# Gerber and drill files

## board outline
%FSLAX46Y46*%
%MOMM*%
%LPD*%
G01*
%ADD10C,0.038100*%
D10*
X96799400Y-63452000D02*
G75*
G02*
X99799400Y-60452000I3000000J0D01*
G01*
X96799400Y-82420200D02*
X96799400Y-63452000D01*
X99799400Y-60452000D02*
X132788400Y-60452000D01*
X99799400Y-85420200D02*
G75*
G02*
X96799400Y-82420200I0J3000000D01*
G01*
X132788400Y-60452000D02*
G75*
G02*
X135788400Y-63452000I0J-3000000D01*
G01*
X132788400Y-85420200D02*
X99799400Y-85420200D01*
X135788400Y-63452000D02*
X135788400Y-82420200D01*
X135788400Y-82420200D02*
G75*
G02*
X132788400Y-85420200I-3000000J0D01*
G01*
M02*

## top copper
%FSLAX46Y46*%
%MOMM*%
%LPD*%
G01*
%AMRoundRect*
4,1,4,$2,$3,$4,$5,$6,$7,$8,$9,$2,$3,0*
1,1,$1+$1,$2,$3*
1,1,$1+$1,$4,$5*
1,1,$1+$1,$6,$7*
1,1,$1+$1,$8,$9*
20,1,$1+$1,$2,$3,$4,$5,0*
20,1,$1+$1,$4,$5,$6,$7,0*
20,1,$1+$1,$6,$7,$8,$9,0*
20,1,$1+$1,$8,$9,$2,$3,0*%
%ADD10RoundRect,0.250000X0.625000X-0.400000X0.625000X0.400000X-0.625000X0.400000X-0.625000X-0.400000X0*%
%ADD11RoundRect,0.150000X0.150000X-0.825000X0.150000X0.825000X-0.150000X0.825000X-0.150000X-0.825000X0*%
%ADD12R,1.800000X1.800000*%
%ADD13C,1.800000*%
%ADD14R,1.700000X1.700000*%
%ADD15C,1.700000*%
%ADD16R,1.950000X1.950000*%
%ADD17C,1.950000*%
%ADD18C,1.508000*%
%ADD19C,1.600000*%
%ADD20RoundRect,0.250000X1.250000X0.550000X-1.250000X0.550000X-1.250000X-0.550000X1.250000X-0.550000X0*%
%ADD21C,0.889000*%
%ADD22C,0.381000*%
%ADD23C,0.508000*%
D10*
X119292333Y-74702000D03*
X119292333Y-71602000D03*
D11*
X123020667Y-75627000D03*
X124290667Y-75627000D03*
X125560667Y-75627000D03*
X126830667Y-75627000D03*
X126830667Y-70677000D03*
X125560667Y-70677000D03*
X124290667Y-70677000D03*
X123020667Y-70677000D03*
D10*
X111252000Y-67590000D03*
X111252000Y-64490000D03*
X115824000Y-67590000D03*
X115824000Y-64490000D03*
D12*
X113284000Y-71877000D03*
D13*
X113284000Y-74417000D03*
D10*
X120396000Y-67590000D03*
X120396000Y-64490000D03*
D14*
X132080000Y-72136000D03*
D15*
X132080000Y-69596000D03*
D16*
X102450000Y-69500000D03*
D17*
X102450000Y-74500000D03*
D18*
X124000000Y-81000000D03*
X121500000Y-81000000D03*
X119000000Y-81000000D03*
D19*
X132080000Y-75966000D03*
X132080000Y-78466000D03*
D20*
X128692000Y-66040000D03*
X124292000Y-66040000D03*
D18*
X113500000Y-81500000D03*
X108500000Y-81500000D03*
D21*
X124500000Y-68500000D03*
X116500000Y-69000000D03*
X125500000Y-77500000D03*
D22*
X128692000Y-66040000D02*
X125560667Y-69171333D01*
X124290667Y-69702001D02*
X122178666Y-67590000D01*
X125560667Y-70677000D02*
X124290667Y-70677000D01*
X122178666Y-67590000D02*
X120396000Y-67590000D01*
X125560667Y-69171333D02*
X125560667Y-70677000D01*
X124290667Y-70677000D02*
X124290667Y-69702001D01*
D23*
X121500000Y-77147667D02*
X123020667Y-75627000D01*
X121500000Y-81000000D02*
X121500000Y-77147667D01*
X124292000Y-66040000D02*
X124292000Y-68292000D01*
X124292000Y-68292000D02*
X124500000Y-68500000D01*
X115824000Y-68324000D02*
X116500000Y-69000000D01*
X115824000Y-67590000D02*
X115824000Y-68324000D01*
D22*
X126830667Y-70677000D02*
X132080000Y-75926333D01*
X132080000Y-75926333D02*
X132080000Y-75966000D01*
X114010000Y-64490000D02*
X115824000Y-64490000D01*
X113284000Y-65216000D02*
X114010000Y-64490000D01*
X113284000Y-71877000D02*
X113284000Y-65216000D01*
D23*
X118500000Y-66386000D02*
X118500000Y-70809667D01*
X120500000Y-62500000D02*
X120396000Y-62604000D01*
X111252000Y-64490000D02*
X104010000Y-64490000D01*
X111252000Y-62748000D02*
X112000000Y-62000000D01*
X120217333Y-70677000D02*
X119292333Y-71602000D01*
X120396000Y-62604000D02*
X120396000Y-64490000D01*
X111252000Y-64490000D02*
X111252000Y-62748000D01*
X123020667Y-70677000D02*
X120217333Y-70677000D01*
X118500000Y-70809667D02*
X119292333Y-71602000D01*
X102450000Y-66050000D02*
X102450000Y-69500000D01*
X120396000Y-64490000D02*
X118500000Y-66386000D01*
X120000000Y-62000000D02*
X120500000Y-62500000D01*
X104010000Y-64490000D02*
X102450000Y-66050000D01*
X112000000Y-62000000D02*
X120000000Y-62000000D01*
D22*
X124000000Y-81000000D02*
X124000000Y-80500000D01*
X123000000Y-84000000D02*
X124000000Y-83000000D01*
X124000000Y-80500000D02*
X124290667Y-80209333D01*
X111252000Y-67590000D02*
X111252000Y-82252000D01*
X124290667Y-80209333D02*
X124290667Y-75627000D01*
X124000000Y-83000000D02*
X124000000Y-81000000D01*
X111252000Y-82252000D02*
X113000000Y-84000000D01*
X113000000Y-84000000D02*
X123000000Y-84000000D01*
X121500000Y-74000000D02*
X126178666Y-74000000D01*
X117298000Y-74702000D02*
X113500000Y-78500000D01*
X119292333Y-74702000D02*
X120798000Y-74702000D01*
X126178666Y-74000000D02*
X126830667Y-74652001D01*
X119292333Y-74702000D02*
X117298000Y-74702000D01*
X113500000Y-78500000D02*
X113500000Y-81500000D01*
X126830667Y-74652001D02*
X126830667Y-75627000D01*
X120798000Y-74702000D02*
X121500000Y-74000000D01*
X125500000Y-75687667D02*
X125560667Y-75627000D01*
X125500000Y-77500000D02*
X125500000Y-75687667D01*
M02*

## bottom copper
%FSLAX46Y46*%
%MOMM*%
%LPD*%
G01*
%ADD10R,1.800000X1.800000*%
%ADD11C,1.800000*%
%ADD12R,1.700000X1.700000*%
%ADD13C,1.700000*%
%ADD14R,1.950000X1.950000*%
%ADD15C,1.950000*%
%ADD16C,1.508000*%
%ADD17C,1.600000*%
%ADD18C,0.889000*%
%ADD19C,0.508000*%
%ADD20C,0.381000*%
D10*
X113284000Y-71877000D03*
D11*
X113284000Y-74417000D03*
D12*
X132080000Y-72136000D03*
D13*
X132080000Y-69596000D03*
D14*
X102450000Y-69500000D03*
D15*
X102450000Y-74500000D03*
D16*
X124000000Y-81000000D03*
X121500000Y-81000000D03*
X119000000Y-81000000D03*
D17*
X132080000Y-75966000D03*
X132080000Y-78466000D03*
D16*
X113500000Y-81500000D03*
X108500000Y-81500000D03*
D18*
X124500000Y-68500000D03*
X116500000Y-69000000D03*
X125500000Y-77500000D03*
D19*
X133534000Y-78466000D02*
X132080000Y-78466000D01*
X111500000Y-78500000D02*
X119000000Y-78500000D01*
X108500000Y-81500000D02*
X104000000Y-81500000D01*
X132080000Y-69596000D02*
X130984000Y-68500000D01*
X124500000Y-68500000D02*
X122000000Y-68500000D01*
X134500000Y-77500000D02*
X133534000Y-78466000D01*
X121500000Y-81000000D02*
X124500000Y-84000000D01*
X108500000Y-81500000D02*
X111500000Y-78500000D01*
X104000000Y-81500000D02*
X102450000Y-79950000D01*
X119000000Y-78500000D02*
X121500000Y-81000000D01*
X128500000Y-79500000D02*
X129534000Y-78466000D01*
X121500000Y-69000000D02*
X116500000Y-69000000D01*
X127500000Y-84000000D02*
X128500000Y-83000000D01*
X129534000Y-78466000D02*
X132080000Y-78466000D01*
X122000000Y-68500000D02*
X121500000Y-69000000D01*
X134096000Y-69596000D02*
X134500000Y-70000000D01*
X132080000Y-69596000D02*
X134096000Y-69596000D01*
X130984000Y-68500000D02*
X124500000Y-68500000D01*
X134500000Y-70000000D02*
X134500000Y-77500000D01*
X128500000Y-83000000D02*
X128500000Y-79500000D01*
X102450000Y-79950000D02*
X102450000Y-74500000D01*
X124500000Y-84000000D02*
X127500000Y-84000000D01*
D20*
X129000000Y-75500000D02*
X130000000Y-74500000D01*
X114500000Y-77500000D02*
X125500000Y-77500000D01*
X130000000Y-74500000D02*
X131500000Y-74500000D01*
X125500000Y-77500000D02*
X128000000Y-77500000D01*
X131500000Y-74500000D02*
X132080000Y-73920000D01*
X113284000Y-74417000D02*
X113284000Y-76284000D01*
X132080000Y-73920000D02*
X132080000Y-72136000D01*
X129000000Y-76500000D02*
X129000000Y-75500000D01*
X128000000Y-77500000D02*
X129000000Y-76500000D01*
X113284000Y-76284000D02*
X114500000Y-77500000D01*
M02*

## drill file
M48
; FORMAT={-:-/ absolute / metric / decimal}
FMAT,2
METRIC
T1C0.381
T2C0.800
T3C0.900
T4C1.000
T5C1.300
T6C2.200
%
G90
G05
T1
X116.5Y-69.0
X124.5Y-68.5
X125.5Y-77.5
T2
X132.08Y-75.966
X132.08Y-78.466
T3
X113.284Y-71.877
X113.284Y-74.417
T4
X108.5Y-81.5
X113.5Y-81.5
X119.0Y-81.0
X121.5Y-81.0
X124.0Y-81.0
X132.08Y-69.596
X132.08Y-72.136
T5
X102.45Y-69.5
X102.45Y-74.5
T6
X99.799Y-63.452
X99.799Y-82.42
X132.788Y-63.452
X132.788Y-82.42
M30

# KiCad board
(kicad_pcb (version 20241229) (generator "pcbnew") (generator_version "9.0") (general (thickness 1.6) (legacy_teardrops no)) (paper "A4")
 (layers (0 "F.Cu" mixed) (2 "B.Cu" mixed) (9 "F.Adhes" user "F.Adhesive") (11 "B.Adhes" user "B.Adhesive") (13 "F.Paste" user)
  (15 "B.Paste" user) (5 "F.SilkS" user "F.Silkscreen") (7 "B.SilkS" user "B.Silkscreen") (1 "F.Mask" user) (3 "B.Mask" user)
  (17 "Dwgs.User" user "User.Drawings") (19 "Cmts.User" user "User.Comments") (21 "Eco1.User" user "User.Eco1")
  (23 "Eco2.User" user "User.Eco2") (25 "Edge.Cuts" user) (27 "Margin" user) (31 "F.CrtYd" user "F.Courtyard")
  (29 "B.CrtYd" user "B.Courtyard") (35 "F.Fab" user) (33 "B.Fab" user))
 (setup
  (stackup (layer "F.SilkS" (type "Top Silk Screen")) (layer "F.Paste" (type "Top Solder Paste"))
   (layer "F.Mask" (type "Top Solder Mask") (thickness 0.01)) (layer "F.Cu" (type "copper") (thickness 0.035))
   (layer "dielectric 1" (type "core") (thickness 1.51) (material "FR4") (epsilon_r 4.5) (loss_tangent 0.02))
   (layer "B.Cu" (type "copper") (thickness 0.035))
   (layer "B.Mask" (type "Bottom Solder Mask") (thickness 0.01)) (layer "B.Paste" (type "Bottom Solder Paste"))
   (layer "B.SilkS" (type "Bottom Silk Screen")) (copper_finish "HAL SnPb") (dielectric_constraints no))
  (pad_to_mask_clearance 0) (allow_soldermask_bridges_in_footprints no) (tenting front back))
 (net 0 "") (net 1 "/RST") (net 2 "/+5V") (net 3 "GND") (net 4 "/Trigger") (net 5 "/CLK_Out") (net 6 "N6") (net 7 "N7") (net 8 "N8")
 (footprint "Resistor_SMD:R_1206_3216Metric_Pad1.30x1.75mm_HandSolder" (layer "F.Cu") (at 119.292333 73.152 90)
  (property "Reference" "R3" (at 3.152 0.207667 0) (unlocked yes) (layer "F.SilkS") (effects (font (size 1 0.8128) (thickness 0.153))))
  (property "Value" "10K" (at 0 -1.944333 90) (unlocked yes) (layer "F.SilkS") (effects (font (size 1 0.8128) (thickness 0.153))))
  (pad "1" smd roundrect (at -1.55 0 90) (size 1.3 1.75) (layers "F.Cu" "F.Mask" "F.Paste") (roundrect_rratio 0.192308) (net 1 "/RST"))
  (pad "2" smd roundrect (at 1.55 0 90) (size 1.3 1.75) (layers "F.Cu" "F.Mask" "F.Paste") (roundrect_rratio 0.192308) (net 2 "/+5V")))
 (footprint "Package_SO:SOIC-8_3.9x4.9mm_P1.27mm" (layer "F.Cu") (at 124.925667 73.152 90)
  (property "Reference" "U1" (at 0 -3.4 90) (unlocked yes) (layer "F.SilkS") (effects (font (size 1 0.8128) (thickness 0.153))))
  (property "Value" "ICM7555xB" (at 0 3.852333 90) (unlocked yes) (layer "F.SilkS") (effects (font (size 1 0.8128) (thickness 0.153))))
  (pad "1" smd roundrect (at -2.475 -1.905 90) (size 1.95 0.6) (layers "F.Cu" "F.Mask" "F.Paste") (roundrect_rratio 0.25) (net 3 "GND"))
  (pad "2" smd roundrect (at -2.475 -0.635 90) (size 1.95 0.6) (layers "F.Cu" "F.Mask" "F.Paste") (roundrect_rratio 0.25) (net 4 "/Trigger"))
  (pad "3" smd roundrect (at -2.475 0.635 90) (size 1.95 0.6) (layers "F.Cu" "F.Mask" "F.Paste") (roundrect_rratio 0.25) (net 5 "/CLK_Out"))
  (pad "4" smd roundrect (at -2.475 1.905 90) (size 1.95 0.6) (layers "F.Cu" "F.Mask" "F.Paste") (roundrect_rratio 0.25) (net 1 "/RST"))
  (pad "5" smd roundrect (at 2.475 1.905 90) (size 1.95 0.6) (layers "F.Cu" "F.Mask" "F.Paste") (roundrect_rratio 0.25) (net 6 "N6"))
  (pad "6" smd roundrect (at 2.475 0.635 90) (size 1.95 0.6) (layers "F.Cu" "F.Mask" "F.Paste") (roundrect_rratio 0.25) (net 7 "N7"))
  (pad "7" smd roundrect (at 2.475 -0.635 90) (size 1.95 0.6) (layers "F.Cu" "F.Mask" "F.Paste") (roundrect_rratio 0.25) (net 7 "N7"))
  (pad "8" smd roundrect (at 2.475 -1.905 90) (size 1.95 0.6) (layers "F.Cu" "F.Mask" "F.Paste") (roundrect_rratio 0.25) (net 2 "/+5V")))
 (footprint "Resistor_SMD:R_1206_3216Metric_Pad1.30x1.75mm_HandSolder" (layer "F.Cu") (at 111.252 66.04 90)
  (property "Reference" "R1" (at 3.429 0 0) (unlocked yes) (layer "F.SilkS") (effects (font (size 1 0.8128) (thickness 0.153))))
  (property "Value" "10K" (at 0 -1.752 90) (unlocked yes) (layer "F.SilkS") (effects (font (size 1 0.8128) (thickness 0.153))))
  (pad "1" smd roundrect (at -1.55 0 90) (size 1.3 1.75) (layers "F.Cu" "F.Mask" "F.Paste") (roundrect_rratio 0.192308) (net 4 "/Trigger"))
  (pad "2" smd roundrect (at 1.55 0 90) (size 1.3 1.75) (layers "F.Cu" "F.Mask" "F.Paste") (roundrect_rratio 0.192308) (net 2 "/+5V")))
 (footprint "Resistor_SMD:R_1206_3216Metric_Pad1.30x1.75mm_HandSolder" (layer "F.Cu") (at 115.824 66.04 90)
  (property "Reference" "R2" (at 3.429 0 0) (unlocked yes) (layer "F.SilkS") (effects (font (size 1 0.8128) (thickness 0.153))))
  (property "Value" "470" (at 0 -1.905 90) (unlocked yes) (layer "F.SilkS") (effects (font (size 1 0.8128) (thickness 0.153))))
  (pad "1" smd roundrect (at -1.55 0 90) (size 1.3 1.75) (layers "F.Cu" "F.Mask" "F.Paste") (roundrect_rratio 0.192308) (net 3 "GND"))
  (pad "2" smd roundrect (at 1.55 0 90) (size 1.3 1.75) (layers "F.Cu" "F.Mask" "F.Paste") (roundrect_rratio 0.192308) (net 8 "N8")))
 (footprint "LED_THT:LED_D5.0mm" (layer "F.Cu") (at 113.284 71.877 -90)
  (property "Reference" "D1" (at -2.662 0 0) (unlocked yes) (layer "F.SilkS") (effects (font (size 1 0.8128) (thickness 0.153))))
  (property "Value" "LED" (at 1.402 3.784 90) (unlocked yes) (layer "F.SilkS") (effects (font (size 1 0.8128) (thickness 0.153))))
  (pad "1" thru_hole rect (at 0 0 270) (size 1.8 1.8) (drill 0.9) (layers "*.Cu" "*.Mask") (remove_unused_layers no) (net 8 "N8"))
  (pad "2" thru_hole circle (at 2.54 0 270) (size 1.8 1.8) (drill 0.9) (layers "*.Cu" "*.Mask") (remove_unused_layers no) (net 5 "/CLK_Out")))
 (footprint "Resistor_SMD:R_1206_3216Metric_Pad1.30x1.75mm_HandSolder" (layer "F.Cu") (at 120.396 66.04 90)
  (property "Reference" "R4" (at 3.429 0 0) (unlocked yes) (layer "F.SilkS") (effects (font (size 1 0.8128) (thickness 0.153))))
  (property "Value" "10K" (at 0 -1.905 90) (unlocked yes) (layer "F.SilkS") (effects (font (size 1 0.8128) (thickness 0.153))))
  (pad "1" smd roundrect (at -1.55 0 90) (size 1.3 1.75) (layers "F.Cu" "F.Mask" "F.Paste") (roundrect_rratio 0.192308) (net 7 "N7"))
  (pad "2" smd roundrect (at 1.55 0 90) (size 1.3 1.75) (layers "F.Cu" "F.Mask" "F.Paste") (roundrect_rratio 0.192308) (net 2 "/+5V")))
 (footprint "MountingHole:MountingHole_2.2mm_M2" (layer "F.Cu") (at 99.7994 63.452)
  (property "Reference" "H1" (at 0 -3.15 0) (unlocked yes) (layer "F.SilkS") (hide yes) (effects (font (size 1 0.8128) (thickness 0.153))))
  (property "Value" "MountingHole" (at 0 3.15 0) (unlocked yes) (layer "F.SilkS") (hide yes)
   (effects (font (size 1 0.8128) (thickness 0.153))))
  (pad "" np_thru_hole circle (at 0 0) (size 2.2 2.2) (drill 2.2) (layers "*.Cu" "*.Mask")))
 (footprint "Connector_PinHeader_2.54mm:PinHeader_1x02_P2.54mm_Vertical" (layer "F.Cu") (at 132.08 72.136 180)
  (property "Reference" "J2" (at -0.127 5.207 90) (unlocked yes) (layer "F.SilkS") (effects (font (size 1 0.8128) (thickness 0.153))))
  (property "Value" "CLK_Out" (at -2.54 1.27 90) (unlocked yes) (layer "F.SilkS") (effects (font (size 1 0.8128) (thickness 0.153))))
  (pad "1" thru_hole rect (at 0 0 180) (size 1.7 1.7) (drill 1) (layers "*.Cu" "*.Mask") (remove_unused_layers no) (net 5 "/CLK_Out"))
  (pad "2" thru_hole circle (at 0 2.54 180) (size 1.7 1.7) (drill 1) (layers "*.Cu" "*.Mask") (remove_unused_layers no) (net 3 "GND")))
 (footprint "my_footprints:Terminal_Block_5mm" (layer "F.Cu") (at 102.45 72 -90)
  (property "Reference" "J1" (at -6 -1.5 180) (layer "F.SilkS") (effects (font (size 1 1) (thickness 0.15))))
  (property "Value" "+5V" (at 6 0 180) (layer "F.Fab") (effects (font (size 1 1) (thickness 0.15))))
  (pad "1" thru_hole rect (at -2.5 0 270) (size 1.95 1.95) (drill 1.3) (layers "*.Cu" "*.Mask") (remove_unused_layers no) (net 2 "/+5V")
   (solder_mask_margin 0.102))
  (pad "2" thru_hole circle (at 2.5 0 270) (size 1.95 1.95) (drill 1.3) (layers "*.Cu" "*.Mask") (remove_unused_layers no) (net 3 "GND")
   (solder_mask_margin 0.102)))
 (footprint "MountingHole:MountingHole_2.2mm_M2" (layer "F.Cu") (at 132.7884 82.4202)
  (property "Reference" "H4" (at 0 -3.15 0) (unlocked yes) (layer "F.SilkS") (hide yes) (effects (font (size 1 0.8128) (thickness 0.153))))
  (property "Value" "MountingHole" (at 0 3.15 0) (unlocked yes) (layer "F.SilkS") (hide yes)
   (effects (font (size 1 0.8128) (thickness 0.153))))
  (pad "" np_thru_hole circle (at 0 0) (size 2.2 2.2) (drill 2.2) (layers "*.Cu" "*.Mask")))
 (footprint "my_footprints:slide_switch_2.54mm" (layer "F.Cu") (at 121.5 81 180)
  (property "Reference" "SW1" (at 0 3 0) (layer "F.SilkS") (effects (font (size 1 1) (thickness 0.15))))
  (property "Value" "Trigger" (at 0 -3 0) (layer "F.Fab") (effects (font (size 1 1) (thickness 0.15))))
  (pad "1" thru_hole circle (at -2.5 0 180) (size 1.508 1.508) (drill 1) (layers "*.Cu" "*.Mask") (remove_unused_layers no)
   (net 4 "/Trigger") (solder_mask_margin 0.102))
  (pad "2" thru_hole circle (at 0 0 180) (size 1.508 1.508) (drill 1) (layers "*.Cu" "*.Mask") (remove_unused_layers no) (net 3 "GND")
   (solder_mask_margin 0.102))
  (pad "3" thru_hole circle (at 2.5 0 180) (size 1.508 1.508) (drill 1) (layers "*.Cu" "*.Mask") (remove_unused_layers no)
   (solder_mask_margin 0.102)))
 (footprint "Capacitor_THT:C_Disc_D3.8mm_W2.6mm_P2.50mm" (layer "F.Cu") (at 132.08 75.966 -90)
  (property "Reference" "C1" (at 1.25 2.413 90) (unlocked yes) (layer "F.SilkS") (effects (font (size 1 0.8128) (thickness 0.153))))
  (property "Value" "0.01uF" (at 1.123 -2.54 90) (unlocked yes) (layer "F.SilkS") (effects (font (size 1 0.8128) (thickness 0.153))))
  (pad "1" thru_hole circle (at 0 0 270) (size 1.6 1.6) (drill 0.8) (layers "*.Cu" "*.Mask") (remove_unused_layers no) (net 6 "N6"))
  (pad "2" thru_hole circle (at 2.5 0 270) (size 1.6 1.6) (drill 0.8) (layers "*.Cu" "*.Mask") (remove_unused_layers no) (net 3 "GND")))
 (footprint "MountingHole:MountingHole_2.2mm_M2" (layer "F.Cu") (at 132.7884 63.452)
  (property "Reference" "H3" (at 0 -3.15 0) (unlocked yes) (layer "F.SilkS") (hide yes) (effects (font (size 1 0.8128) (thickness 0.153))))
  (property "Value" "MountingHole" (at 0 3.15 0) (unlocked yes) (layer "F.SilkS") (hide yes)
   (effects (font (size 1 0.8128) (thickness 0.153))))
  (pad "" np_thru_hole circle (at 0 0) (size 2.2 2.2) (drill 2.2) (layers "*.Cu" "*.Mask")))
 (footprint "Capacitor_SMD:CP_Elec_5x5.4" (layer "F.Cu") (at 126.492 66.04 180)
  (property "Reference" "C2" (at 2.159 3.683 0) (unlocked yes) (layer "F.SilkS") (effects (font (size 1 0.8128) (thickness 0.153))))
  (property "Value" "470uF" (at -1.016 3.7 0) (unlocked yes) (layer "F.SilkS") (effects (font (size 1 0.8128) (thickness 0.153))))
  (pad "1" smd roundrect (at -2.2 0 180) (size 3 1.6) (layers "F.Cu" "F.Mask" "F.Paste") (roundrect_rratio 0.15625) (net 7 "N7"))
  (pad "2" smd roundrect (at 2.2 0 180) (size 3 1.6) (layers "F.Cu" "F.Mask" "F.Paste") (roundrect_rratio 0.15625) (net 3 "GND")))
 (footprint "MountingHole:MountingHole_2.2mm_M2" (layer "F.Cu") (at 99.7994 82.4202)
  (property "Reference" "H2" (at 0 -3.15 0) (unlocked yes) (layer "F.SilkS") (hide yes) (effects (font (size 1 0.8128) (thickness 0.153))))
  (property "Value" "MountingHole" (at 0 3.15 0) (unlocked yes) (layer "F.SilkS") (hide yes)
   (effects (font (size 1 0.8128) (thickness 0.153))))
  (pad "" np_thru_hole circle (at 0 0) (size 2.2 2.2) (drill 2.2) (layers "*.Cu" "*.Mask")))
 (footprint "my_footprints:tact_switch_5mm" (layer "F.Cu") (at 111 81.5 180)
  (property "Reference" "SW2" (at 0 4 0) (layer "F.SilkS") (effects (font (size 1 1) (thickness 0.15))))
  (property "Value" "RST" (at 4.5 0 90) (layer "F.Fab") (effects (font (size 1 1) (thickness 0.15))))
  (pad "1" thru_hole circle (at -2.5 0 180) (size 1.508 1.508) (drill 1) (layers "*.Cu" "*.Mask") (remove_unused_layers no) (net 1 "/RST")
   (solder_mask_margin 0.102))
  (pad "2" thru_hole circle (at 2.5 0 180) (size 1.508 1.508) (drill 1) (layers "*.Cu" "*.Mask") (remove_unused_layers no) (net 3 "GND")
   (solder_mask_margin 0.102)))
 (gr_arc (start 96.7994 63.452) (mid 97.67808 61.33068) (end 99.7994 60.452) (stroke (width 0.0381) (type default)) (layer "Edge.Cuts"))
 (gr_line (start 96.7994 82.4202) (end 96.7994 63.452) (stroke (width 0.0381) (type default)) (layer "Edge.Cuts"))
 (gr_line (start 99.7994 60.452) (end 132.7884 60.452) (stroke (width 0.0381) (type default)) (layer "Edge.Cuts"))
 (gr_arc (start 99.7994 85.4202) (mid 97.67808 84.54152) (end 96.7994 82.4202) (stroke (width 0.0381) (type default)) (layer "Edge.Cuts"))
 (gr_arc (start 132.7884 60.452) (mid 134.90972 61.33068) (end 135.7884 63.452) (stroke (width 0.0381) (type default)) (layer "Edge.Cuts"))
 (gr_line (start 132.7884 85.4202) (end 99.7994 85.4202) (stroke (width 0.0381) (type default)) (layer "Edge.Cuts"))
 (gr_line (start 135.7884 63.452) (end 135.7884 82.4202) (stroke (width 0.0381) (type default)) (layer "Edge.Cuts"))
 (gr_arc (start 135.7884 82.4202) (mid 134.90972 84.54152) (end 132.7884 85.4202) (stroke (width 0.0381) (type default)) (layer "Edge.Cuts"))
 (segment (start 128.692 66.04) (end 125.560667 69.171333) (width 0.381) (layer "F.Cu") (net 7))
 (segment (start 124.290667 69.702001) (end 122.178666 67.59) (width 0.381) (layer "F.Cu") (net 7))
 (segment (start 125.560667 70.677) (end 124.290667 70.677) (width 0.381) (layer "F.Cu") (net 7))
 (segment (start 122.178666 67.59) (end 120.396 67.59) (width 0.381) (layer "F.Cu") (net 7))
 (segment (start 125.560667 69.171333) (end 125.560667 70.677) (width 0.381) (layer "F.Cu") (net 7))
 (segment (start 124.290667 70.677) (end 124.290667 69.702001) (width 0.381) (layer "F.Cu") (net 7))
 (segment (start 121.5 77.147667) (end 123.020667 75.627) (width 0.508) (layer "F.Cu") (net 3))
 (segment (start 121.5 81) (end 121.5 77.147667) (width 0.508) (layer "F.Cu") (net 3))
 (segment (start 124.292 66.04) (end 124.292 68.292) (width 0.508) (layer "F.Cu") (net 3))
 (segment (start 124.292 68.292) (end 124.5 68.5) (width 0.508) (layer "F.Cu") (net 3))
 (segment (start 115.824 68.324) (end 116.5 69) (width 0.508) (layer "F.Cu") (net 3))
 (segment (start 115.824 67.59) (end 115.824 68.324) (width 0.508) (layer "F.Cu") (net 3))
 (via (at 124.5 68.5) (size 0.889) (drill 0.381) (layers "F.Cu" "B.Cu") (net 3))
 (via (at 116.5 69) (size 0.889) (drill 0.381) (layers "F.Cu" "B.Cu") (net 3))
 (segment (start 133.534 78.466) (end 132.08 78.466) (width 0.508) (layer "B.Cu") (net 3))
 (segment (start 111.5 78.5) (end 119 78.5) (width 0.508) (layer "B.Cu") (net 3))
 (segment (start 108.5 81.5) (end 104 81.5) (width 0.508) (layer "B.Cu") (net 3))
 (segment (start 132.08 69.596) (end 130.984 68.5) (width 0.508) (layer "B.Cu") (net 3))
 (segment (start 124.5 68.5) (end 122 68.5) (width 0.508) (layer "B.Cu") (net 3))
 (segment (start 134.5 77.5) (end 133.534 78.466) (width 0.508) (layer "B.Cu") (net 3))
 (segment (start 121.5 81) (end 124.5 84) (width 0.508) (layer "B.Cu") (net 3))
 (segment (start 108.5 81.5) (end 111.5 78.5) (width 0.508) (layer "B.Cu") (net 3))
 (segment (start 104 81.5) (end 102.45 79.95) (width 0.508) (layer "B.Cu") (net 3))
 (segment (start 119 78.5) (end 121.5 81) (width 0.508) (layer "B.Cu") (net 3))
 (segment (start 128.5 79.5) (end 129.534 78.466) (width 0.508) (layer "B.Cu") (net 3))
 (segment (start 121.5 69) (end 116.5 69) (width 0.508) (layer "B.Cu") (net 3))
 (segment (start 127.5 84) (end 128.5 83) (width 0.508) (layer "B.Cu") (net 3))
 (segment (start 129.534 78.466) (end 132.08 78.466) (width 0.508) (layer "B.Cu") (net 3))
 (segment (start 122 68.5) (end 121.5 69) (width 0.508) (layer "B.Cu") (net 3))
 (segment (start 134.096 69.596) (end 134.5 70) (width 0.508) (layer "B.Cu") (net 3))
 (segment (start 132.08 69.596) (end 134.096 69.596) (width 0.508) (layer "B.Cu") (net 3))
 (segment (start 130.984 68.5) (end 124.5 68.5) (width 0.508) (layer "B.Cu") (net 3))
 (segment (start 134.5 70) (end 134.5 77.5) (width 0.508) (layer "B.Cu") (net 3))
 (segment (start 128.5 83) (end 128.5 79.5) (width 0.508) (layer "B.Cu") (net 3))
 (segment (start 102.45 79.95) (end 102.45 74.5) (width 0.508) (layer "B.Cu") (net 3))
 (segment (start 124.5 84) (end 127.5 84) (width 0.508) (layer "B.Cu") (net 3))
 (segment (start 126.830667 70.677) (end 132.08 75.926333) (width 0.381) (layer "F.Cu") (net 6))
 (segment (start 132.08 75.926333) (end 132.08 75.966) (width 0.381) (layer "F.Cu") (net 6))
 (segment (start 114.01 64.49) (end 115.824 64.49) (width 0.381) (layer "F.Cu") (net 8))
 (segment (start 113.284 65.216) (end 114.01 64.49) (width 0.381) (layer "F.Cu") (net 8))
 (segment (start 113.284 71.877) (end 113.284 65.216) (width 0.381) (layer "F.Cu") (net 8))
 (segment (start 118.5 66.386) (end 118.5 70.809667) (width 0.508) (layer "F.Cu") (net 2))
 (segment (start 120.5 62.5) (end 120.396 62.604) (width 0.508) (layer "F.Cu") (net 2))
 (segment (start 111.252 64.49) (end 104.01 64.49) (width 0.508) (layer "F.Cu") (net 2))
 (segment (start 111.252 62.748) (end 112 62) (width 0.508) (layer "F.Cu") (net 2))
 (segment (start 120.217333 70.677) (end 119.292333 71.602) (width 0.508) (layer "F.Cu") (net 2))
 (segment (start 120.396 62.604) (end 120.396 64.49) (width 0.508) (layer "F.Cu") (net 2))
 (segment (start 111.252 64.49) (end 111.252 62.748) (width 0.508) (layer "F.Cu") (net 2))
 (segment (start 123.020667 70.677) (end 120.217333 70.677) (width 0.508) (layer "F.Cu") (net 2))
 (segment (start 118.5 70.809667) (end 119.292333 71.602) (width 0.508) (layer "F.Cu") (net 2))
 (segment (start 102.45 66.05) (end 102.45 69.5) (width 0.508) (layer "F.Cu") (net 2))
 (segment (start 120.396 64.49) (end 118.5 66.386) (width 0.508) (layer "F.Cu") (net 2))
 (segment (start 120 62) (end 120.5 62.5) (width 0.508) (layer "F.Cu") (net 2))
 (segment (start 104.01 64.49) (end 102.45 66.05) (width 0.508) (layer "F.Cu") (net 2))
 (segment (start 112 62) (end 120 62) (width 0.508) (layer "F.Cu") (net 2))
 (segment (start 124 81) (end 124 80.5) (width 0.381) (layer "F.Cu") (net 4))
 (segment (start 123 84) (end 124 83) (width 0.381) (layer "F.Cu") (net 4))
 (segment (start 124 80.5) (end 124.290667 80.209333) (width 0.381) (layer "F.Cu") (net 4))
 (segment (start 111.252 67.59) (end 111.252 82.252) (width 0.381) (layer "F.Cu") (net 4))
 (segment (start 124.290667 80.209333) (end 124.290667 75.627) (width 0.381) (layer "F.Cu") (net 4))
 (segment (start 124 83) (end 124 81) (width 0.381) (layer "F.Cu") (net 4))
 (segment (start 111.252 82.252) (end 113 84) (width 0.381) (layer "F.Cu") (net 4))
 (segment (start 113 84) (end 123 84) (width 0.381) (layer "F.Cu") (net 4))
 (segment (start 121.5 74) (end 126.178666 74) (width 0.381) (layer "F.Cu") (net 1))
 (segment (start 117.298 74.702) (end 113.5 78.5) (width 0.381) (layer "F.Cu") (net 1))
 (segment (start 119.292333 74.702) (end 120.798 74.702) (width 0.381) (layer "F.Cu") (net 1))
 (segment (start 126.178666 74) (end 126.830667 74.652001) (width 0.381) (layer "F.Cu") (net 1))
 (segment (start 119.292333 74.702) (end 117.298 74.702) (width 0.381) (layer "F.Cu") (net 1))
 (segment (start 113.5 78.5) (end 113.5 81.5) (width 0.381) (layer "F.Cu") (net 1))
 (segment (start 126.830667 74.652001) (end 126.830667 75.627) (width 0.381) (layer "F.Cu") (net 1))
 (segment (start 120.798 74.702) (end 121.5 74) (width 0.381) (layer "F.Cu") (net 1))
 (segment (start 125.5 75.687667) (end 125.560667 75.627) (width 0.381) (layer "F.Cu") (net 5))
 (segment (start 125.5 77.5) (end 125.5 75.687667) (width 0.381) (layer "F.Cu") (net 5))
 (via (at 125.5 77.5) (size 0.889) (drill 0.381) (layers "F.Cu" "B.Cu") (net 5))
 (segment (start 129 75.5) (end 130 74.5) (width 0.381) (layer "B.Cu") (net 5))
 (segment (start 114.5 77.5) (end 125.5 77.5) (width 0.381) (layer "B.Cu") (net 5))
 (segment (start 130 74.5) (end 131.5 74.5) (width 0.381) (layer "B.Cu") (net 5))
 (segment (start 125.5 77.5) (end 128 77.5) (width 0.381) (layer "B.Cu") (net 5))
 (segment (start 131.5 74.5) (end 132.08 73.92) (width 0.381) (layer "B.Cu") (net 5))
 (segment (start 113.284 74.417) (end 113.284 76.284) (width 0.381) (layer "B.Cu") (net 5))
 (segment (start 132.08 73.92) (end 132.08 72.136) (width 0.381) (layer "B.Cu") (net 5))
 (segment (start 129 76.5) (end 129 75.5) (width 0.381) (layer "B.Cu") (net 5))
 (segment (start 128 77.5) (end 129 76.5) (width 0.381) (layer "B.Cu") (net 5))
 (segment (start 113.284 76.284) (end 114.5 77.5) (width 0.381) (layer "B.Cu") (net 5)))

